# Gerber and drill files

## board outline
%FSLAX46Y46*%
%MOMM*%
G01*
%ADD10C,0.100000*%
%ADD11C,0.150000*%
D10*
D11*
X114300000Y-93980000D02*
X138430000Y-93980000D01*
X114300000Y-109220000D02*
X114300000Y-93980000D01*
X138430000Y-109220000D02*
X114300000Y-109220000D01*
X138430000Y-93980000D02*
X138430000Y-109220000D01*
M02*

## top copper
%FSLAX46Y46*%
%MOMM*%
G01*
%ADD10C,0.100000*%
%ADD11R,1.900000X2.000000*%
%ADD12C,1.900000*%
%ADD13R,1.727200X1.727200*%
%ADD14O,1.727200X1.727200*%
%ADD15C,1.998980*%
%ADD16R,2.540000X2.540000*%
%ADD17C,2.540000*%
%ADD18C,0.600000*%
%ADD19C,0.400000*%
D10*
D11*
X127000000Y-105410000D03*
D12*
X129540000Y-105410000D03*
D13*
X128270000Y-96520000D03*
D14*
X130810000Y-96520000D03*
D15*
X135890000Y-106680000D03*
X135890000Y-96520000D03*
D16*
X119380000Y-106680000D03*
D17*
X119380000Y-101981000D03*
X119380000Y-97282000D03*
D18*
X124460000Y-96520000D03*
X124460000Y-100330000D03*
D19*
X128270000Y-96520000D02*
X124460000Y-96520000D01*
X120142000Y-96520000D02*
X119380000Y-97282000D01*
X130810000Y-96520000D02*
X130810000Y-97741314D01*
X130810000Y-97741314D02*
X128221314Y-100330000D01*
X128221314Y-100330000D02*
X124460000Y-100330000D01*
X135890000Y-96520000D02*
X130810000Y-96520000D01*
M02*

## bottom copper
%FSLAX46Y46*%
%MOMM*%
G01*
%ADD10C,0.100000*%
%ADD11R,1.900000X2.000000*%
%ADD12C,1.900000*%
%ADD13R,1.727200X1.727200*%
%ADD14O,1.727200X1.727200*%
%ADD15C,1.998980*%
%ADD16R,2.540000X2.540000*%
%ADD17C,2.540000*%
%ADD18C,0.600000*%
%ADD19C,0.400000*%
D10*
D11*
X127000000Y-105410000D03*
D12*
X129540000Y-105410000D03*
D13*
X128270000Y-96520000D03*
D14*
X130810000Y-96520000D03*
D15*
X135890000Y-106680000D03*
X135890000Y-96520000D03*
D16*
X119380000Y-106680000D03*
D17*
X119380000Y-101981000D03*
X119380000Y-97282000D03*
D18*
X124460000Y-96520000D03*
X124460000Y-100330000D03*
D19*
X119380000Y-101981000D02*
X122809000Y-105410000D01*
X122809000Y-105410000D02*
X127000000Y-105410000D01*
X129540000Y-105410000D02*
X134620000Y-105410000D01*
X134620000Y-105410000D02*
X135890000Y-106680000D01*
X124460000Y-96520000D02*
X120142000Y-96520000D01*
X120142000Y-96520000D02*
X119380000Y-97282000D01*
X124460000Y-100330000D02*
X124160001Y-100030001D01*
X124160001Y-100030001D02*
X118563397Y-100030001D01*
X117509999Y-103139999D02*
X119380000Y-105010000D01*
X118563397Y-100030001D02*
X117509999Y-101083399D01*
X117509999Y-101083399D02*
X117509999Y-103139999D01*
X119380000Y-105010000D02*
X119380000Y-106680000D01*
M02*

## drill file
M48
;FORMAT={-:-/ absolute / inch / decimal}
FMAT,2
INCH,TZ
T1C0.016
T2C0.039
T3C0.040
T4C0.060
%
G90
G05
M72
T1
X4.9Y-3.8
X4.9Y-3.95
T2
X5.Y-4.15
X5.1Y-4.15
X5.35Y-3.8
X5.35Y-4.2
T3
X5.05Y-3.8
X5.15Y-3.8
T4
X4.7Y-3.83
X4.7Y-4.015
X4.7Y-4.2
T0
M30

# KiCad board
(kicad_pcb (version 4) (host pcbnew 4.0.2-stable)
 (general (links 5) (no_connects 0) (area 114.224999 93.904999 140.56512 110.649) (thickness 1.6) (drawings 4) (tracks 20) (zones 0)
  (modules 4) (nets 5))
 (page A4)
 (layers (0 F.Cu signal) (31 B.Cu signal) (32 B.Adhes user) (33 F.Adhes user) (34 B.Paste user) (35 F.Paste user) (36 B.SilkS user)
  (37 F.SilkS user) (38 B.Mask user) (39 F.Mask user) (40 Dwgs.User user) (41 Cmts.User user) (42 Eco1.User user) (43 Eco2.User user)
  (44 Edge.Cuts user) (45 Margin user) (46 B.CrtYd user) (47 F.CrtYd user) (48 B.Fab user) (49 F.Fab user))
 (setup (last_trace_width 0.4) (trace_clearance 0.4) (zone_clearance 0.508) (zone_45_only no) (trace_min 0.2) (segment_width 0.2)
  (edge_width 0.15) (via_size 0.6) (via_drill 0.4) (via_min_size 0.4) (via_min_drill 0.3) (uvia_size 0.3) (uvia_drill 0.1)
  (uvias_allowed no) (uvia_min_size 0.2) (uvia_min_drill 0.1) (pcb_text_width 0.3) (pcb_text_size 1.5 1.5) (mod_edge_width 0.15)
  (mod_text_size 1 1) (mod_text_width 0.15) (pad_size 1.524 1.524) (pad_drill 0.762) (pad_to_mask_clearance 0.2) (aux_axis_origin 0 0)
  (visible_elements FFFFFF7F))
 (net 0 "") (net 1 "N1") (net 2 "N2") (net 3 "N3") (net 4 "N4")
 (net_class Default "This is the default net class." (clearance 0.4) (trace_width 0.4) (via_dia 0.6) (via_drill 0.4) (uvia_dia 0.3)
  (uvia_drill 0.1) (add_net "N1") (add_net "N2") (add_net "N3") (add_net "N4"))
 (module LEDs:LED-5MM (layer F.Cu) (at 127 105.41)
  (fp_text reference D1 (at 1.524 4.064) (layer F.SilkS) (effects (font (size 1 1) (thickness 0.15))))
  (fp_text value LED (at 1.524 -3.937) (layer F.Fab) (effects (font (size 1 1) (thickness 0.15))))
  (pad 1 thru_hole rect (at 0 0 90) (size 2 1.9) (drill 1.00076) (layers *.Cu *.Mask F.SilkS) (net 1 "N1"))
  (pad 2 thru_hole circle (at 2.54 0) (size 1.9 1.9) (drill 1.00076) (layers *.Cu *.Mask F.SilkS) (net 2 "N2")))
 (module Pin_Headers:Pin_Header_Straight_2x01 (layer B.Cu) (at 128.27 96.52)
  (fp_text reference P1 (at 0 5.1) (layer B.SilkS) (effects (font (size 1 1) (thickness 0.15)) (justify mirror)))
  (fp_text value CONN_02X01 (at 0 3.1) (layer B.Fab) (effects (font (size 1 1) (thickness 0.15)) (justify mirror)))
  (pad 1 thru_hole rect (at 0 0) (size 1.7272 1.7272) (drill 1.016) (layers *.Cu *.Mask B.SilkS) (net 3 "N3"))
  (pad 2 thru_hole oval (at 2.54 0) (size 1.7272 1.7272) (drill 1.016) (layers *.Cu *.Mask B.SilkS) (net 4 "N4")))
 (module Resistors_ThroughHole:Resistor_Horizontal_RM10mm (layer B.Cu) (at 135.89 106.68 90)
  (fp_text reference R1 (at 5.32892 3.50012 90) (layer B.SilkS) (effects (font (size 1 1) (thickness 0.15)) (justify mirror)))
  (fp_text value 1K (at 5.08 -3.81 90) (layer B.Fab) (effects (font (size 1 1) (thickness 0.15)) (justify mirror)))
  (pad 1 thru_hole circle (at 0 0 90) (size 1.99898 1.99898) (drill 1.00076) (layers *.Cu *.SilkS *.Mask) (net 2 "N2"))
  (pad 2 thru_hole circle (at 10.16 0 90) (size 1.99898 1.99898) (drill 1.00076) (layers *.Cu *.SilkS *.Mask) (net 4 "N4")))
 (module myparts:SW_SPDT (layer F.Cu) (at 119.38 101.981 90)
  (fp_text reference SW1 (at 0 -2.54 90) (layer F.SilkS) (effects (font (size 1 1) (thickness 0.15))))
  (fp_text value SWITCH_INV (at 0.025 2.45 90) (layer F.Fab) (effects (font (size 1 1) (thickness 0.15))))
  (pad 1 thru_hole rect (at -4.699 0 90) (size 2.54 2.54) (drill 1.524) (layers *.Cu *.Mask F.SilkS) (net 4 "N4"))
  (pad 2 thru_hole circle (at 0 0 90) (size 2.54 2.54) (drill 1.524) (layers *.Cu *.Mask F.SilkS) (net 1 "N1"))
  (pad 3 thru_hole circle (at 4.699 0 90) (size 2.54 2.54) (drill 1.524) (layers *.Cu *.Mask F.SilkS) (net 3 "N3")))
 (gr_line (start 114.3 93.98) (end 138.43 93.98) (layer Edge.Cuts) (width 0.15))
 (gr_line (start 114.3 109.22) (end 114.3 93.98) (layer Edge.Cuts) (width 0.15))
 (gr_line (start 138.43 109.22) (end 114.3 109.22) (layer Edge.Cuts) (width 0.15))
 (gr_line (start 138.43 93.98) (end 138.43 109.22) (layer Edge.Cuts) (width 0.15))
 (segment (start 119.38 101.981) (end 122.809 105.41) (width 0.4) (layer B.Cu) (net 1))
 (segment (start 122.809 105.41) (end 127 105.41) (width 0.4) (layer B.Cu) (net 1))
 (segment (start 129.54 105.41) (end 134.62 105.41) (width 0.4) (layer B.Cu) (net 2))
 (segment (start 134.62 105.41) (end 135.89 106.68) (width 0.4) (layer B.Cu) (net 2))
 (segment (start 124.46 96.52) (end 120.142 96.52) (width 0.4) (layer B.Cu) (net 3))
 (segment (start 120.142 96.52) (end 119.38 97.282) (width 0.4) (layer B.Cu) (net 3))
 (segment (start 128.27 96.52) (end 124.46 96.52) (width 0.4) (layer F.Cu) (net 3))
 (via (at 124.46 96.52) (size 0.6) (drill 0.4) (layers F.Cu B.Cu) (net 3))
 (segment (start 120.142 96.52) (end 119.38 97.282) (width 0.4) (layer F.Cu) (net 3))
 (segment (start 124.46 100.33) (end 124.160001 100.030001) (width 0.4) (layer B.Cu) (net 4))
 (segment (start 124.160001 100.030001) (end 118.563397 100.030001) (width 0.4) (layer B.Cu) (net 4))
 (segment (start 117.509999 103.139999) (end 119.38 105.01) (width 0.4) (layer B.Cu) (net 4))
 (segment (start 118.563397 100.030001) (end 117.509999 101.083399) (width 0.4) (layer B.Cu) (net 4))
 (segment (start 117.509999 101.083399) (end 117.509999 103.139999) (width 0.4) (layer B.Cu) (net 4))
 (segment (start 119.38 105.01) (end 119.38 106.68) (width 0.4) (layer B.Cu) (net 4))
 (segment (start 130.81 96.52) (end 130.81 97.741314) (width 0.4) (layer F.Cu) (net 4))
 (segment (start 130.81 97.741314) (end 128.221314 100.33) (width 0.4) (layer F.Cu) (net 4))
 (segment (start 128.221314 100.33) (end 124.46 100.33) (width 0.4) (layer F.Cu) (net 4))
 (via (at 124.46 100.33) (size 0.6) (drill 0.4) (layers F.Cu B.Cu) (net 4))
 (segment (start 135.89 96.52) (end 130.81 96.52) (width 0.4) (layer F.Cu) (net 4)))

